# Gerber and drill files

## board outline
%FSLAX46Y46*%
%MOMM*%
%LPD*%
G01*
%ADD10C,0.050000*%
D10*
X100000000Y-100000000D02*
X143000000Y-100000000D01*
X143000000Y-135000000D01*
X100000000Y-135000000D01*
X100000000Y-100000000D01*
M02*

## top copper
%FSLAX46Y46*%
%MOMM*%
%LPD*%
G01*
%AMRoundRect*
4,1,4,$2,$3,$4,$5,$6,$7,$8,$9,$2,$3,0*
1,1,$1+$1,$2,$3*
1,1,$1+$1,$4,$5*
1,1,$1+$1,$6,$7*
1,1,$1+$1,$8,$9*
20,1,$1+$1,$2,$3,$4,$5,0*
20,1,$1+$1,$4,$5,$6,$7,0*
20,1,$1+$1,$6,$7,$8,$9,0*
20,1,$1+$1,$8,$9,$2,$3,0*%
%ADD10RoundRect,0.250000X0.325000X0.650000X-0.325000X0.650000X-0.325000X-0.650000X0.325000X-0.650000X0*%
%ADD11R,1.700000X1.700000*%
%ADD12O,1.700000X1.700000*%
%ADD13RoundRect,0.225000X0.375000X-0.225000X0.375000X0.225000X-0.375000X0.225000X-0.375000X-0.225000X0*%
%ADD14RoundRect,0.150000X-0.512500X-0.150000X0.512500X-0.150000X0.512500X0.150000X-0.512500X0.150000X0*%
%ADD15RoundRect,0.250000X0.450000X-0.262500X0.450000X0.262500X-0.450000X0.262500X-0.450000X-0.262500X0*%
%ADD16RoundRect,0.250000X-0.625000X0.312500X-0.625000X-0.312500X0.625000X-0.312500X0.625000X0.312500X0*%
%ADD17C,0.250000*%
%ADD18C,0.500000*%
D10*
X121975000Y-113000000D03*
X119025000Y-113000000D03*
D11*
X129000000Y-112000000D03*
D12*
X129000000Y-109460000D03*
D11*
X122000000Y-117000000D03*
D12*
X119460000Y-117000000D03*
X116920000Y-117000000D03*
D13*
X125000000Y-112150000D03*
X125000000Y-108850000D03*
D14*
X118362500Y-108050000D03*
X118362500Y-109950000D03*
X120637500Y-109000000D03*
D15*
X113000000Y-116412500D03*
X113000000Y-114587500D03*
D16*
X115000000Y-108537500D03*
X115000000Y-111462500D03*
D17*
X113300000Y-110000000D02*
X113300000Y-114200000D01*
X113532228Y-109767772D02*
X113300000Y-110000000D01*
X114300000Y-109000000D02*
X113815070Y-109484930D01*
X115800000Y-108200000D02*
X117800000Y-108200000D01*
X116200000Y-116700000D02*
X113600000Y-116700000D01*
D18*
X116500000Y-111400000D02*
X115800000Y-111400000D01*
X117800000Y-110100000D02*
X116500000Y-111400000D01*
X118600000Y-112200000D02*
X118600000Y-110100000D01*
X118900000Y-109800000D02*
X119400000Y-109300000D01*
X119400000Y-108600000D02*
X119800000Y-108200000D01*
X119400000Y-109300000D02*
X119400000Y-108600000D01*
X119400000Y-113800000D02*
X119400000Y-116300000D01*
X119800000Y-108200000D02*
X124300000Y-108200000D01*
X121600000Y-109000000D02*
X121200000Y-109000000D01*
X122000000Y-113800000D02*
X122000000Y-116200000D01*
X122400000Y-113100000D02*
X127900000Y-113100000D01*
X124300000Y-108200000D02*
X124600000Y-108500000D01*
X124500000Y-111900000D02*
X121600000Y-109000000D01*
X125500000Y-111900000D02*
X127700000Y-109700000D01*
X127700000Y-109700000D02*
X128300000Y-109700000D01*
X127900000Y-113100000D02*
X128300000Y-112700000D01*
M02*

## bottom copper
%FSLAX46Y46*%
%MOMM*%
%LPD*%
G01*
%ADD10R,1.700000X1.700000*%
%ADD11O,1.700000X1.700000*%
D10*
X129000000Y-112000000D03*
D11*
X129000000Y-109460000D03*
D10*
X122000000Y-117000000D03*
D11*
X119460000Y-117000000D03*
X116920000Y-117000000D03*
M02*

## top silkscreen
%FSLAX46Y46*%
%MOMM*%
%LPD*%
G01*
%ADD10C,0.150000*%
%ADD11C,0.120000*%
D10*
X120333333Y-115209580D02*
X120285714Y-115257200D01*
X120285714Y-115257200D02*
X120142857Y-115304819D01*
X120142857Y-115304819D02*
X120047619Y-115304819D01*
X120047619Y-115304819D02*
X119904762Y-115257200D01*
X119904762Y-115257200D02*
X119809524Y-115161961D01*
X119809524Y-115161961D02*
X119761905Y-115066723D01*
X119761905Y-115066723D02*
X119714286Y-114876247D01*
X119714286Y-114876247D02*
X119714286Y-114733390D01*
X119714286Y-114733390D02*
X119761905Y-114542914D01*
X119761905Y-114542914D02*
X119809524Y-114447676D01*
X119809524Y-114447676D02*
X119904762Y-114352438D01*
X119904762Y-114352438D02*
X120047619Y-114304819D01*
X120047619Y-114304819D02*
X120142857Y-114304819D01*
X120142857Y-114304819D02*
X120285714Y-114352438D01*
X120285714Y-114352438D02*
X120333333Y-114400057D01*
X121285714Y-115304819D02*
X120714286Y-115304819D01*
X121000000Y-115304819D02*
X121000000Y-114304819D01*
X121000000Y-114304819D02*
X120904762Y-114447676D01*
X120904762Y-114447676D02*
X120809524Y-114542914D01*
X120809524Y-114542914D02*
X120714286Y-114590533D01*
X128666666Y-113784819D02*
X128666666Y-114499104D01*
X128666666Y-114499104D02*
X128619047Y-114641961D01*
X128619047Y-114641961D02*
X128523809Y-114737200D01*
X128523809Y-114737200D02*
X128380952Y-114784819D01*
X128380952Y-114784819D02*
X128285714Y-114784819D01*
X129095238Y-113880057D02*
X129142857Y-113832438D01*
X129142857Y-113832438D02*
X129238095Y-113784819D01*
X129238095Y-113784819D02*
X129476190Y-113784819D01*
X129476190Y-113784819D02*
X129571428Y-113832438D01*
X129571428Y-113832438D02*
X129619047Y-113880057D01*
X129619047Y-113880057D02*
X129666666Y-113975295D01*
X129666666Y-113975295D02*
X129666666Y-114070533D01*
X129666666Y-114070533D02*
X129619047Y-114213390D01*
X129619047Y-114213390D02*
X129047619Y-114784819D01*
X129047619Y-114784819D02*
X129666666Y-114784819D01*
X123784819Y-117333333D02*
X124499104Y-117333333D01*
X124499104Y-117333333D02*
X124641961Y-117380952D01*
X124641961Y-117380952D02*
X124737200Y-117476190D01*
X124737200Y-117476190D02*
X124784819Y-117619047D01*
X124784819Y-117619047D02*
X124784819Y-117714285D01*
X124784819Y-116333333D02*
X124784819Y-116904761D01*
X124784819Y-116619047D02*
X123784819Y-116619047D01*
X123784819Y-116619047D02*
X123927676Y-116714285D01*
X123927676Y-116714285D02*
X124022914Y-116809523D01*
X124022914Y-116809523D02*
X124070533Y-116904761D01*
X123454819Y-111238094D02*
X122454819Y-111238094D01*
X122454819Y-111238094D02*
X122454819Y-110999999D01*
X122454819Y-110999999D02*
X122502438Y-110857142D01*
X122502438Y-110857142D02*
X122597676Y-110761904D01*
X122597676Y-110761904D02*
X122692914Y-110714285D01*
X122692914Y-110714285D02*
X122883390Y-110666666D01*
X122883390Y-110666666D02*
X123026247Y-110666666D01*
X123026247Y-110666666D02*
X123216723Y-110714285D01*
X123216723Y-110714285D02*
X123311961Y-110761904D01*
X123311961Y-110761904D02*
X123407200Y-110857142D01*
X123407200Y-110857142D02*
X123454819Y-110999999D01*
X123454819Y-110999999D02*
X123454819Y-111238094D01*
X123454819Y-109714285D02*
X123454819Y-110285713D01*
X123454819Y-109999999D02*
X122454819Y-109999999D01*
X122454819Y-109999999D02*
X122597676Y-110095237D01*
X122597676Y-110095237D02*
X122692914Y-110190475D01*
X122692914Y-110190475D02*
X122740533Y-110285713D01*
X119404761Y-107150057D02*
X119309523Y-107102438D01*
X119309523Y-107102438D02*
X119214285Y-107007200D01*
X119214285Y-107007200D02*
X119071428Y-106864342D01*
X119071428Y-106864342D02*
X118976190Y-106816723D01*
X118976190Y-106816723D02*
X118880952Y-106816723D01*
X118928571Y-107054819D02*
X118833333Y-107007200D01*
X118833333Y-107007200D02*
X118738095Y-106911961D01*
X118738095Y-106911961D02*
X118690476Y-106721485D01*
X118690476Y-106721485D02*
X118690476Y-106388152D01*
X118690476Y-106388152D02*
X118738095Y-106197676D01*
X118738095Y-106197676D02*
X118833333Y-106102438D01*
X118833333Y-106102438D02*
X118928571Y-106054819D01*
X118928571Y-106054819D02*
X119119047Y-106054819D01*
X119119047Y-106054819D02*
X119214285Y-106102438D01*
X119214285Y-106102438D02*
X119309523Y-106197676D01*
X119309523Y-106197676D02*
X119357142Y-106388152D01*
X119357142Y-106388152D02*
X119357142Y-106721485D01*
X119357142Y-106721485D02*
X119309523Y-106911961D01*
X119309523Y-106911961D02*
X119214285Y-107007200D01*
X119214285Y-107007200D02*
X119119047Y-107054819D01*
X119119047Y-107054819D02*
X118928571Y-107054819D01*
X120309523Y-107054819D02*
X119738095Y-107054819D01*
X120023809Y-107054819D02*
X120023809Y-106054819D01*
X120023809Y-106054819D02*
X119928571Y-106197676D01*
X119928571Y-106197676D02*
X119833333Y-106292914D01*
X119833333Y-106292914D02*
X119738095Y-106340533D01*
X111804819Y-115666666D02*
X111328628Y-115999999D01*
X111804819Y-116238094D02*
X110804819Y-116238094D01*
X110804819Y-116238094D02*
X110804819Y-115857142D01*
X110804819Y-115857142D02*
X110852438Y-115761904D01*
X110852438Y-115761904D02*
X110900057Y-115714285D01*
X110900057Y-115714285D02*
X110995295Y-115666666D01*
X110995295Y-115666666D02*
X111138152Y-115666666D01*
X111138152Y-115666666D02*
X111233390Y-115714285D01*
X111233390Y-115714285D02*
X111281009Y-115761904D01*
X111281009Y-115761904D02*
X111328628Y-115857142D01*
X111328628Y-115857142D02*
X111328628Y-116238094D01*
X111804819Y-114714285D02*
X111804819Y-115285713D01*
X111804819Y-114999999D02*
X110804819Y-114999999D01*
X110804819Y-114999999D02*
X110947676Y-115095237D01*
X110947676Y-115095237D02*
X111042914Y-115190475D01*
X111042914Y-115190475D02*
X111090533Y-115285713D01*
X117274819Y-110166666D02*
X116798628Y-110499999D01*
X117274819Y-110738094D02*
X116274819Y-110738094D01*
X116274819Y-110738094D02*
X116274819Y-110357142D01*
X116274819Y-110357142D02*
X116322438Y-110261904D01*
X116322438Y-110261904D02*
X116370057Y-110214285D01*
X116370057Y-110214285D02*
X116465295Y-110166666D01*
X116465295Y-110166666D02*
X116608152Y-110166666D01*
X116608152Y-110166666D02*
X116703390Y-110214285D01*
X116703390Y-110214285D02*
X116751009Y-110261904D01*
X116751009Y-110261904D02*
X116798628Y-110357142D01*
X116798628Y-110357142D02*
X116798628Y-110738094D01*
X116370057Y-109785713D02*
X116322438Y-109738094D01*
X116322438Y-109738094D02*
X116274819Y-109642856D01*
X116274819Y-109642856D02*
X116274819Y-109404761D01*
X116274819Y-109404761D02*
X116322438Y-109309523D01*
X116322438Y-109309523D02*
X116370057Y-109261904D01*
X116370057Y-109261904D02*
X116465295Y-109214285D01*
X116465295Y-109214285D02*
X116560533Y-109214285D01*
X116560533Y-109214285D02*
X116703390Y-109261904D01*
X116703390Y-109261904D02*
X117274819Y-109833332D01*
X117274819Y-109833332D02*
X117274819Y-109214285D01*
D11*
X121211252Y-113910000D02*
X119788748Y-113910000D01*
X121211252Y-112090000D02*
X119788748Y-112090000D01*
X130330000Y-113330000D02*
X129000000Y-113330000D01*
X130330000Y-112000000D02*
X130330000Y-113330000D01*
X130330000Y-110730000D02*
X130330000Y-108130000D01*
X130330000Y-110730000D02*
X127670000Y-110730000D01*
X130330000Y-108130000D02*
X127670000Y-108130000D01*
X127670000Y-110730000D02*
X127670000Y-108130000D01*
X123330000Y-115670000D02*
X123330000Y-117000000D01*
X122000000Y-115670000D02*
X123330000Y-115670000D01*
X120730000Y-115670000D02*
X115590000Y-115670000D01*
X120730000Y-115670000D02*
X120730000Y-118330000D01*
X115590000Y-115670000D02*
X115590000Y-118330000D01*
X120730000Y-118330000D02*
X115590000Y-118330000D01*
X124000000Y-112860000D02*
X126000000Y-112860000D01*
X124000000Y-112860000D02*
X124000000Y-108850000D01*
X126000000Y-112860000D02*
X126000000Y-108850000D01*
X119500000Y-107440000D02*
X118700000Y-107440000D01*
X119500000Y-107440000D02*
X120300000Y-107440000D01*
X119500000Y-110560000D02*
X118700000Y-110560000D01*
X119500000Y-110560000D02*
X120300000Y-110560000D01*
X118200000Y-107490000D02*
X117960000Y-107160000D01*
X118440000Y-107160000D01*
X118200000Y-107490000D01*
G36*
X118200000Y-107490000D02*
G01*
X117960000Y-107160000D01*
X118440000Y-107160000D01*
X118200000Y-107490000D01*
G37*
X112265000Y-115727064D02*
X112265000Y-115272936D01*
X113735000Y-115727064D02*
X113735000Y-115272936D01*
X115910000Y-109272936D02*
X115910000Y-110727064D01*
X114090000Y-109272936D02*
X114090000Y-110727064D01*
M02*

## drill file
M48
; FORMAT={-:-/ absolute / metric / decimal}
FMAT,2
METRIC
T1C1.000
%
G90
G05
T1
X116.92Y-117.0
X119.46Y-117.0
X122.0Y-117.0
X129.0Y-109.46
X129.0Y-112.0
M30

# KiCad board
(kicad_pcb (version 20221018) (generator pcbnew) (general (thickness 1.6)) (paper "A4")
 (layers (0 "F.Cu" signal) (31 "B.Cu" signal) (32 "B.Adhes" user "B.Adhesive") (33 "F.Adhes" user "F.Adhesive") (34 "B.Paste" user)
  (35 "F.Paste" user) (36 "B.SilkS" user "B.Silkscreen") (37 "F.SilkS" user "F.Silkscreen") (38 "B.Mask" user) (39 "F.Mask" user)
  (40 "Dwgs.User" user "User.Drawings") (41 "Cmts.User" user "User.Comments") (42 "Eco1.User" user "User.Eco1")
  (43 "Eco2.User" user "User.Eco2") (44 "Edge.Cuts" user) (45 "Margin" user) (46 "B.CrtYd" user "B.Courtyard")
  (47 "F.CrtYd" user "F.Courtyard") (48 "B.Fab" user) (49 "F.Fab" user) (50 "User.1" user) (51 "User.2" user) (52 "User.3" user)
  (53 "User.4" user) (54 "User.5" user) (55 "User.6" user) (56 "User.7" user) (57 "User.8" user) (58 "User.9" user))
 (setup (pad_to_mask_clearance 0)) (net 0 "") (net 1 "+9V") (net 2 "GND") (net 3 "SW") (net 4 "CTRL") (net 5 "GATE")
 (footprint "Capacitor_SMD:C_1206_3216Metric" (layer "F.Cu") (at 120.5 113 180)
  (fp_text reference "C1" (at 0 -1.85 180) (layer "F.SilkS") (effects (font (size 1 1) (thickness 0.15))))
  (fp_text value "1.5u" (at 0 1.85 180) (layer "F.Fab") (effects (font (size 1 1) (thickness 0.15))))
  (fp_line (start -0.711252 -0.91) (end 0.711252 -0.91) (stroke (width 0.12) (type solid)) (layer "F.SilkS"))
  (fp_line (start -0.711252 0.91) (end 0.711252 0.91) (stroke (width 0.12) (type solid)) (layer "F.SilkS"))
  (pad "1" smd roundrect (at -1.475 0 180) (size 1.15 1.8) (layers "F.Cu" "F.Paste" "F.Mask") (roundrect_rratio 0.217391) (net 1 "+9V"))
  (pad "2" smd roundrect (at 1.475 0 180) (size 1.15 1.8) (layers "F.Cu" "F.Paste" "F.Mask") (roundrect_rratio 0.217391) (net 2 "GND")))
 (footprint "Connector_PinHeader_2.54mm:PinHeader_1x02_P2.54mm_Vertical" (layer "F.Cu") (at 129 112 180)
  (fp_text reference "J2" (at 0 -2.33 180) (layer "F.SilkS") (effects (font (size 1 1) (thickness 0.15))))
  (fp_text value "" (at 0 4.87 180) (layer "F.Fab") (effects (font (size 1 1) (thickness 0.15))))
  (fp_line (start -1.33 -1.33) (end 0 -1.33) (stroke (width 0.12) (type solid)) (layer "F.SilkS"))
  (fp_line (start -1.33 0) (end -1.33 -1.33) (stroke (width 0.12) (type solid)) (layer "F.SilkS"))
  (fp_line (start -1.33 1.27) (end -1.33 3.87) (stroke (width 0.12) (type solid)) (layer "F.SilkS"))
  (fp_line (start -1.33 1.27) (end 1.33 1.27) (stroke (width 0.12) (type solid)) (layer "F.SilkS"))
  (fp_line (start -1.33 3.87) (end 1.33 3.87) (stroke (width 0.12) (type solid)) (layer "F.SilkS"))
  (fp_line (start 1.33 1.27) (end 1.33 3.87) (stroke (width 0.12) (type solid)) (layer "F.SilkS"))
  (pad "1" thru_hole rect (at 0 0 180) (size 1.7 1.7) (drill 1) (layers "*.Cu" "*.Mask") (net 1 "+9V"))
  (pad "2" thru_hole oval (at 0 2.54 180) (size 1.7 1.7) (drill 1) (layers "*.Cu" "*.Mask") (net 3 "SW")))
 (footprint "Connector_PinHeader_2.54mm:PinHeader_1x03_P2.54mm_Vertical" (layer "F.Cu") (at 122 117 -90)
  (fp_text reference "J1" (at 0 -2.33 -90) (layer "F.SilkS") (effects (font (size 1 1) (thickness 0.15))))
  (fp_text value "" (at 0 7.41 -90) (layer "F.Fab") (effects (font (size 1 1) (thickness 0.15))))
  (fp_line (start -1.33 -1.33) (end 0 -1.33) (stroke (width 0.12) (type solid)) (layer "F.SilkS"))
  (fp_line (start -1.33 0) (end -1.33 -1.33) (stroke (width 0.12) (type solid)) (layer "F.SilkS"))
  (fp_line (start -1.33 1.27) (end -1.33 6.41) (stroke (width 0.12) (type solid)) (layer "F.SilkS"))
  (fp_line (start -1.33 1.27) (end 1.33 1.27) (stroke (width 0.12) (type solid)) (layer "F.SilkS"))
  (fp_line (start -1.33 6.41) (end 1.33 6.41) (stroke (width 0.12) (type solid)) (layer "F.SilkS"))
  (fp_line (start 1.33 1.27) (end 1.33 6.41) (stroke (width 0.12) (type solid)) (layer "F.SilkS"))
  (pad "1" thru_hole rect (at 0 0 270) (size 1.7 1.7) (drill 1) (layers "*.Cu" "*.Mask") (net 1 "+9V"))
  (pad "2" thru_hole oval (at 0 2.54 270) (size 1.7 1.7) (drill 1) (layers "*.Cu" "*.Mask") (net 2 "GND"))
  (pad "3" thru_hole oval (at 0 5.08 270) (size 1.7 1.7) (drill 1) (layers "*.Cu" "*.Mask") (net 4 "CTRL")))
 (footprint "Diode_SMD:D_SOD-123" (layer "F.Cu") (at 125 110.5 90)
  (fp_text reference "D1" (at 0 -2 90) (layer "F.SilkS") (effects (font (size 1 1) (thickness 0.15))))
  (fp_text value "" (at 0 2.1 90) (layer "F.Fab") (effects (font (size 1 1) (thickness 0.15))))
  (fp_line (start -2.36 -1) (end -2.36 1) (stroke (width 0.12) (type solid)) (layer "F.SilkS"))
  (fp_line (start -2.36 -1) (end 1.65 -1) (stroke (width 0.12) (type solid)) (layer "F.SilkS"))
  (fp_line (start -2.36 1) (end 1.65 1) (stroke (width 0.12) (type solid)) (layer "F.SilkS"))
  (pad "1" smd roundrect (at -1.65 0 90) (size 0.9 1.2) (layers "F.Cu" "F.Paste" "F.Mask") (roundrect_rratio 0.25) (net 3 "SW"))
  (pad "2" smd roundrect (at 1.65 0 90) (size 0.9 1.2) (layers "F.Cu" "F.Paste" "F.Mask") (roundrect_rratio 0.25) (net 2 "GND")))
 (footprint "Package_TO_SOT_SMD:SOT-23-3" (layer "F.Cu") (at 119.5 109)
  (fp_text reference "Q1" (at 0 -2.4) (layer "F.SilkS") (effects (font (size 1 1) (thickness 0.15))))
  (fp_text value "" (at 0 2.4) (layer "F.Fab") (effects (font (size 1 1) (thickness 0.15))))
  (fp_line (start 0 -1.56) (end -0.8 -1.56) (stroke (width 0.12) (type solid)) (layer "F.SilkS"))
  (fp_line (start 0 -1.56) (end 0.8 -1.56) (stroke (width 0.12) (type solid)) (layer "F.SilkS"))
  (fp_line (start 0 1.56) (end -0.8 1.56) (stroke (width 0.12) (type solid)) (layer "F.SilkS"))
  (fp_line (start 0 1.56) (end 0.8 1.56) (stroke (width 0.12) (type solid)) (layer "F.SilkS"))
  (fp_poly
   (pts (xy -1.3 -1.51) (xy -1.54 -1.84) (xy -1.06 -1.84) (xy -1.3 -1.51)) (stroke (width 0.12) (type solid)) (fill solid) (layer "F.SilkS"))
  (pad "1" smd roundrect (at -1.1375 -0.95) (size 1.325 0.6) (layers "F.Cu" "F.Paste" "F.Mask") (roundrect_rratio 0.25) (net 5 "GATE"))
  (pad "2" smd roundrect (at -1.1375 0.95) (size 1.325 0.6) (layers "F.Cu" "F.Paste" "F.Mask") (roundrect_rratio 0.25) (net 2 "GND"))
  (pad "3" smd roundrect (at 1.1375 0) (size 1.325 0.6) (layers "F.Cu" "F.Paste" "F.Mask") (roundrect_rratio 0.25) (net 3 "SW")))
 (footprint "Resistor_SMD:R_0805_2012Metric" (layer "F.Cu") (at 113 115.5 90)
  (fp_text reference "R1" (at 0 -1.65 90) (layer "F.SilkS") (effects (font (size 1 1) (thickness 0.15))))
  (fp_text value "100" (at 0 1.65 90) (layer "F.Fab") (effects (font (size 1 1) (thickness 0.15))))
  (fp_line (start -0.227064 -0.735) (end 0.227064 -0.735) (stroke (width 0.12) (type solid)) (layer "F.SilkS"))
  (fp_line (start -0.227064 0.735) (end 0.227064 0.735) (stroke (width 0.12) (type solid)) (layer "F.SilkS"))
  (pad "1" smd roundrect (at -0.9125 0 90) (size 1.025 1.4) (layers "F.Cu" "F.Paste" "F.Mask") (roundrect_rratio 0.243902) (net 4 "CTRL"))
  (pad "2" smd roundrect (at 0.9125 0 90) (size 1.025 1.4) (layers "F.Cu" "F.Paste" "F.Mask") (roundrect_rratio 0.243902) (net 5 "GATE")))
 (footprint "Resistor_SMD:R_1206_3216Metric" (layer "F.Cu") (at 115 110 -90)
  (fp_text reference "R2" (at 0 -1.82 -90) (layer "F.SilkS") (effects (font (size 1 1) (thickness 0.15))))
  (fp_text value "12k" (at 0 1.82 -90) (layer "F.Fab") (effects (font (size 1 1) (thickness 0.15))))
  (fp_line (start -0.727064 -0.91) (end 0.727064 -0.91) (stroke (width 0.12) (type solid)) (layer "F.SilkS"))
  (fp_line (start -0.727064 0.91) (end 0.727064 0.91) (stroke (width 0.12) (type solid)) (layer "F.SilkS"))
  (pad "1" smd roundrect (at -1.4625 0 270) (size 1.125 1.75) (layers "F.Cu" "F.Paste" "F.Mask") (roundrect_rratio 0.222222) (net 5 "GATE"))
  (pad "2" smd roundrect (at 1.4625 0 270) (size 1.125 1.75) (layers "F.Cu" "F.Paste" "F.Mask") (roundrect_rratio 0.222222) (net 2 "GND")))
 (gr_rect (start 100 100) (end 143 135) (stroke (width 0.05) (type default)) (fill none) (layer "Edge.Cuts"))
 (segment (start 113.3 110) (end 113.3 114.2) (width 0.25) (layer "F.Cu") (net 5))
 (segment (start 113.532228 109.767772) (end 113.3 110) (width 0.25) (layer "F.Cu") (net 5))
 (segment (start 114.3 109) (end 113.81507 109.48493) (width 0.25) (layer "F.Cu") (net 5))
 (segment (start 115.8 108.2) (end 117.8 108.2) (width 0.25) (layer "F.Cu") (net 5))
 (segment (start 116.2 116.7) (end 113.6 116.7) (width 0.25) (layer "F.Cu") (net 4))
 (segment (start 116.5 111.4) (end 115.8 111.4) (width 0.5) (layer "F.Cu") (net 2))
 (segment (start 117.8 110.1) (end 116.5 111.4) (width 0.5) (layer "F.Cu") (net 2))
 (segment (start 118.6 112.2) (end 118.6 110.1) (width 0.5) (layer "F.Cu") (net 2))
 (segment (start 118.9 109.8) (end 119.4 109.3) (width 0.5) (layer "F.Cu") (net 2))
 (segment (start 119.4 108.6) (end 119.8 108.2) (width 0.5) (layer "F.Cu") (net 2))
 (segment (start 119.4 109.3) (end 119.4 108.6) (width 0.5) (layer "F.Cu") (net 2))
 (segment (start 119.4 113.8) (end 119.4 116.3) (width 0.5) (layer "F.Cu") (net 2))
 (segment (start 119.8 108.2) (end 124.3 108.2) (width 0.5) (layer "F.Cu") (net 2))
 (segment (start 121.6 109) (end 121.2 109) (width 0.5) (layer "F.Cu") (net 3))
 (segment (start 122 113.8) (end 122 116.2) (width 0.5) (layer "F.Cu") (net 1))
 (segment (start 122.4 113.1) (end 127.9 113.1) (width 0.5) (layer "F.Cu") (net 1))
 (segment (start 124.3 108.2) (end 124.6 108.5) (width 0.5) (layer "F.Cu") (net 2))
 (segment (start 124.5 111.9) (end 121.6 109) (width 0.5) (layer "F.Cu") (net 3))
 (segment (start 125.5 111.9) (end 127.7 109.7) (width 0.5) (layer "F.Cu") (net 3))
 (segment (start 127.7 109.7) (end 128.3 109.7) (width 0.5) (layer "F.Cu") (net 3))
 (segment (start 127.9 113.1) (end 128.3 112.7) (width 0.5) (layer "F.Cu") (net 1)))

